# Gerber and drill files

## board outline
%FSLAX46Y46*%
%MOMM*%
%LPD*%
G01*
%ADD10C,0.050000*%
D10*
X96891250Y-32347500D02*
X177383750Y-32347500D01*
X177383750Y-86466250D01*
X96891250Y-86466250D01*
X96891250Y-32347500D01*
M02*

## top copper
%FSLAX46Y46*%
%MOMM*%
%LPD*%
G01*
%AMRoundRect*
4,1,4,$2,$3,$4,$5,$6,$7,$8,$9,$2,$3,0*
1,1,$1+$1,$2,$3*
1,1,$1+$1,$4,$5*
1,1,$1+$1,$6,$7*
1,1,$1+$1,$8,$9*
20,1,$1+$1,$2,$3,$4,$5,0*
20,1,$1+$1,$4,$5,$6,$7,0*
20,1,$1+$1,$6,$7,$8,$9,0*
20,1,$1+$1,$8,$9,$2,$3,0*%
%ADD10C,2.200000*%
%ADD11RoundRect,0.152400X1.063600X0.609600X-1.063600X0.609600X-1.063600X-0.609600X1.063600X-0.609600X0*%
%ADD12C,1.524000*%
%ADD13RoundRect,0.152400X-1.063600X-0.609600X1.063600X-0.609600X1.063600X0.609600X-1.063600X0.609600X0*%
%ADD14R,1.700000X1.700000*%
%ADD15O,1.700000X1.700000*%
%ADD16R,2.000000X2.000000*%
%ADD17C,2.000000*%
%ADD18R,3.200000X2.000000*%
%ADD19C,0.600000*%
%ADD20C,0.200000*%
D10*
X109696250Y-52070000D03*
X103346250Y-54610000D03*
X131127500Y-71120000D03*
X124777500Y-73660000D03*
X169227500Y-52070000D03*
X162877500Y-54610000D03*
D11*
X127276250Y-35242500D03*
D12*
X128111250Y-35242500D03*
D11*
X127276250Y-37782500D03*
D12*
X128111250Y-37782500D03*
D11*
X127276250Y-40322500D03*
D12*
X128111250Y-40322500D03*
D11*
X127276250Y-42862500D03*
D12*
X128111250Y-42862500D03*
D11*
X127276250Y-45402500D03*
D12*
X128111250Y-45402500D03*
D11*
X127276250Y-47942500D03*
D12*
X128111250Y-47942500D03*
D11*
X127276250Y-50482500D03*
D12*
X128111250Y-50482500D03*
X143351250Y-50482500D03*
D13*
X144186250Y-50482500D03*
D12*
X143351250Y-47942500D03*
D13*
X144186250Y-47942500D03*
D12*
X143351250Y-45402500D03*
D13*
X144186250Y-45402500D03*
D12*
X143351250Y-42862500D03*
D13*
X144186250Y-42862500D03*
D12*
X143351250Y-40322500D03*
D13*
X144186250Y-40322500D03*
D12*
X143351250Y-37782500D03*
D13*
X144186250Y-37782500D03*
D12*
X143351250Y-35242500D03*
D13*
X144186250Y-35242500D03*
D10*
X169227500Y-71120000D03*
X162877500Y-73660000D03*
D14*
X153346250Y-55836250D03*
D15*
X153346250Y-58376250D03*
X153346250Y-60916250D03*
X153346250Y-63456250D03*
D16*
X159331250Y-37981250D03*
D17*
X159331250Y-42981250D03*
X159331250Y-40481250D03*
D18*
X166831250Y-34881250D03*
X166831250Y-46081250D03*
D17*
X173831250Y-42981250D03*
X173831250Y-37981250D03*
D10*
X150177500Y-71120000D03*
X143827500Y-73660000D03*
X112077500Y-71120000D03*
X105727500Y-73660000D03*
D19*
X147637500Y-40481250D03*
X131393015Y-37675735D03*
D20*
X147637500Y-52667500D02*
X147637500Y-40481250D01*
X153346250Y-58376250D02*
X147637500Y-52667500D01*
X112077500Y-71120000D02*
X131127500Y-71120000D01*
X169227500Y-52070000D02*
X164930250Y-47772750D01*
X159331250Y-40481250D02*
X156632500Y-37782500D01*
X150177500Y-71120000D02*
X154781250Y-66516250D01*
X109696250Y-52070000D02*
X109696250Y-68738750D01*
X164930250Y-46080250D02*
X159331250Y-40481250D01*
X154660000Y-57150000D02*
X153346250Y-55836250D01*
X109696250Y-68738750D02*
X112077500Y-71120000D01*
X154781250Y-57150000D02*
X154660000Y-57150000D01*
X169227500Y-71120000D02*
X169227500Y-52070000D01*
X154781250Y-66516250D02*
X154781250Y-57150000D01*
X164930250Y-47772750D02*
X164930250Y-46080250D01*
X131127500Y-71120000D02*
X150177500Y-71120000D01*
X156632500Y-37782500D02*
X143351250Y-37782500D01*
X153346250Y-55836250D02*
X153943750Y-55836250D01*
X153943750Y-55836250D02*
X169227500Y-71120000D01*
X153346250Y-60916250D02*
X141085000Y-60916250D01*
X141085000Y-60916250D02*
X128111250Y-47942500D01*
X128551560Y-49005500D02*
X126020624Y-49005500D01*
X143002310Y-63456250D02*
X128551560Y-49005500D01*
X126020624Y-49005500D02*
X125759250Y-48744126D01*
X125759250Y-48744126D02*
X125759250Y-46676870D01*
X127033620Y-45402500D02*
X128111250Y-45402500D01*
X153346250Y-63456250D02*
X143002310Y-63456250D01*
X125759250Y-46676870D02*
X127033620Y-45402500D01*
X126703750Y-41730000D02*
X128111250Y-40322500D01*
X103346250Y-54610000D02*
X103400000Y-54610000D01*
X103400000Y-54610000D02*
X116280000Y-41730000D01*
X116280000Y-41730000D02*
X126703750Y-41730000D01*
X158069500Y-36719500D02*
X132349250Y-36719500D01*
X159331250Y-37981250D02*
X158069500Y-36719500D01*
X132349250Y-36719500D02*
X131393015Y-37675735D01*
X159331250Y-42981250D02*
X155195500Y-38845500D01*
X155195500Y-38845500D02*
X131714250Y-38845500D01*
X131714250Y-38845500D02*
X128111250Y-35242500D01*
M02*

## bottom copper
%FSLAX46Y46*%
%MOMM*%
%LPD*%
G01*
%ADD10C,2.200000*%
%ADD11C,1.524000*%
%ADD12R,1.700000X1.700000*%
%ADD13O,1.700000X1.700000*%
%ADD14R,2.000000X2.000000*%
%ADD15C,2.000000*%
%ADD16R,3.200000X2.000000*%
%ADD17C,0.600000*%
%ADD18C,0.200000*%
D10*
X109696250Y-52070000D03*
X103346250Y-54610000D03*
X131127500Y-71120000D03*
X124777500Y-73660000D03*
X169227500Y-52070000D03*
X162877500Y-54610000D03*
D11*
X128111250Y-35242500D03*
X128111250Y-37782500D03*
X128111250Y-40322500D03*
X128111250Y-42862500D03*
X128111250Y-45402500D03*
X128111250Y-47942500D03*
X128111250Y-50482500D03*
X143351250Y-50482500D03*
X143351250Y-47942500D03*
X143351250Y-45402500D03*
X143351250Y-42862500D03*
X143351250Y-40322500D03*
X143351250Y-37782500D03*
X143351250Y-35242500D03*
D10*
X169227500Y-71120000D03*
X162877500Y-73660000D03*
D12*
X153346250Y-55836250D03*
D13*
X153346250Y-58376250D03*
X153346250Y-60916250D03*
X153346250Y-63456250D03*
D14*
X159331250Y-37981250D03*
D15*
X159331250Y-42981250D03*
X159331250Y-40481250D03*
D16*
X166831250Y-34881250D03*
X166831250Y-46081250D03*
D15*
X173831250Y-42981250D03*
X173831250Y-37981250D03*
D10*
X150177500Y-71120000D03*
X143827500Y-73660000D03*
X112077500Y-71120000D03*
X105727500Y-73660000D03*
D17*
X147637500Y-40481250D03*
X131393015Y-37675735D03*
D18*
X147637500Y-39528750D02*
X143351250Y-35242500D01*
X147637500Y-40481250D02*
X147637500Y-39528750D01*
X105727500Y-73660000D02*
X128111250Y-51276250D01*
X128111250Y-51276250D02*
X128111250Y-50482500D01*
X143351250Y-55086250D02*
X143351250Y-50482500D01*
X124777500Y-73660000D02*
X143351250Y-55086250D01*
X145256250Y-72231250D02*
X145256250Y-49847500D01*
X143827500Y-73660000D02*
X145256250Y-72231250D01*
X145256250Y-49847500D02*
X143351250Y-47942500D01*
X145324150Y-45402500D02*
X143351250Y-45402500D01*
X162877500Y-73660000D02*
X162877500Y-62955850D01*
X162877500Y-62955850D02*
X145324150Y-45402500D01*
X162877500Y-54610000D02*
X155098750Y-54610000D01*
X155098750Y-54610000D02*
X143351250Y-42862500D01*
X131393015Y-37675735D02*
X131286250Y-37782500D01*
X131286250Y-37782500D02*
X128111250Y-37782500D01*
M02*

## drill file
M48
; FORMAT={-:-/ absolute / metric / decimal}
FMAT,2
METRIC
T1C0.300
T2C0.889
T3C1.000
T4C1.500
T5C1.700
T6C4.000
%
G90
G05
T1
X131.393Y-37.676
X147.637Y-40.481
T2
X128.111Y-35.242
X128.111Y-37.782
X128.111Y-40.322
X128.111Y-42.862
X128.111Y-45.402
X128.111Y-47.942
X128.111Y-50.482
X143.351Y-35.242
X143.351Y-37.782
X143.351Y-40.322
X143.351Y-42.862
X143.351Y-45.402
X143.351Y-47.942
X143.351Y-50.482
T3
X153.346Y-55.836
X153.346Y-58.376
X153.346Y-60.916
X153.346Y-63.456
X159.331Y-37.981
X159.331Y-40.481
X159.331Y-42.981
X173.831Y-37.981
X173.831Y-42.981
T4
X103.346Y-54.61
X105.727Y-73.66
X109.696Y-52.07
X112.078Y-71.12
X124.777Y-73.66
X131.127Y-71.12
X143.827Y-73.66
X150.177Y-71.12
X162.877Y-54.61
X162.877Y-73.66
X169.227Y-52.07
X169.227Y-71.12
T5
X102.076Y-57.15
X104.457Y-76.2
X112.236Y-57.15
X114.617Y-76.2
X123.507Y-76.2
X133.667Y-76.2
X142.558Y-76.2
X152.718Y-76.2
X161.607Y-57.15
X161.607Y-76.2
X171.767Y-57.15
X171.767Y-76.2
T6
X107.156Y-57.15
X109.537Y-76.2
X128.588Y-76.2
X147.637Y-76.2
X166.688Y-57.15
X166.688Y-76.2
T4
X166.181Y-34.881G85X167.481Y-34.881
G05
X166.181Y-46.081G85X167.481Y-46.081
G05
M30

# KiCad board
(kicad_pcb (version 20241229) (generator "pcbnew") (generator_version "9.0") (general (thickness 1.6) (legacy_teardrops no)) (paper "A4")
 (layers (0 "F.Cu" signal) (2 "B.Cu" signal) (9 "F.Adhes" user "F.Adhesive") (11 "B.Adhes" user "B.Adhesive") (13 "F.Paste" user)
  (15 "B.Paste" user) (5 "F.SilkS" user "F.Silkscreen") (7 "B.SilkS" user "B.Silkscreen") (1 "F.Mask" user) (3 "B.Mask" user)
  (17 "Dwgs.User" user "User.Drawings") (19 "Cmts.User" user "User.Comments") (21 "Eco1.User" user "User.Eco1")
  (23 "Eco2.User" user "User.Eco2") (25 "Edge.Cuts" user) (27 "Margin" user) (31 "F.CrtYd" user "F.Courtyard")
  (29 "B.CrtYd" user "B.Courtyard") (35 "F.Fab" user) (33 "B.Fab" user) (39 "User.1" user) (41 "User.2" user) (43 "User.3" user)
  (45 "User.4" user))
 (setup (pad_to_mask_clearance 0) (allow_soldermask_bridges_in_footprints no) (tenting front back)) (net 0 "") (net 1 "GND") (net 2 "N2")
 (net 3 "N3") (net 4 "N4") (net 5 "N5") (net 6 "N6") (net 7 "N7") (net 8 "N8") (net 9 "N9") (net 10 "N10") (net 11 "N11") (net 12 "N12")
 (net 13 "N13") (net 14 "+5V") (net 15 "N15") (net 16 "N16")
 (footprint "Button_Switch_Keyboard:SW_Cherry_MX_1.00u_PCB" (layer "F.Cu") (at 109.69625 52.07)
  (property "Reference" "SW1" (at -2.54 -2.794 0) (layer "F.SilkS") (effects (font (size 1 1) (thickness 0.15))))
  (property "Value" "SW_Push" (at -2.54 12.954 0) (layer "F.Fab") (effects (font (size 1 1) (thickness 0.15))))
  (pad "" np_thru_hole circle (at -7.62 5.08) (size 1.7 1.7) (drill 1.7) (layers "*.Cu" "*.Mask"))
  (pad "" np_thru_hole circle (at -2.54 5.08) (size 4 4) (drill 4) (layers "*.Cu" "*.Mask"))
  (pad "" np_thru_hole circle (at 2.54 5.08) (size 1.7 1.7) (drill 1.7) (layers "*.Cu" "*.Mask"))
  (pad "1" thru_hole circle (at 0 0) (size 2.2 2.2) (drill 1.5) (layers "*.Cu" "*.Mask") (remove_unused_layers no) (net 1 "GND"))
  (pad "2" thru_hole circle (at -6.35 2.54) (size 2.2 2.2) (drill 1.5) (layers "*.Cu" "*.Mask") (remove_unused_layers no) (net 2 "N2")))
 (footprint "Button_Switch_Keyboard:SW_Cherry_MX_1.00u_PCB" (layer "F.Cu") (at 131.1275 71.12)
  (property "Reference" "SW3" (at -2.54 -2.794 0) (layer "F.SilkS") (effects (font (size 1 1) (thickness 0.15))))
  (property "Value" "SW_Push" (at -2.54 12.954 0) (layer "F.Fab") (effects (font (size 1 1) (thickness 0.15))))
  (pad "" np_thru_hole circle (at -7.62 5.08) (size 1.7 1.7) (drill 1.7) (layers "*.Cu" "*.Mask"))
  (pad "" np_thru_hole circle (at -2.54 5.08) (size 4 4) (drill 4) (layers "*.Cu" "*.Mask"))
  (pad "" np_thru_hole circle (at 2.54 5.08) (size 1.7 1.7) (drill 1.7) (layers "*.Cu" "*.Mask"))
  (pad "1" thru_hole circle (at 0 0) (size 2.2 2.2) (drill 1.5) (layers "*.Cu" "*.Mask") (remove_unused_layers no) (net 1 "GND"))
  (pad "2" thru_hole circle (at -6.35 2.54) (size 2.2 2.2) (drill 1.5) (layers "*.Cu" "*.Mask") (remove_unused_layers no) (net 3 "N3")))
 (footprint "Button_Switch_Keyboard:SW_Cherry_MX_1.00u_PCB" (layer "F.Cu") (at 169.2275 52.07)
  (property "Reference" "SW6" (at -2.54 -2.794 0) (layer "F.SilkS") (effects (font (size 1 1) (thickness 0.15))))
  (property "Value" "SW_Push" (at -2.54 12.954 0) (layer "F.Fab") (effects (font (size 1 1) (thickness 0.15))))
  (pad "" np_thru_hole circle (at -7.62 5.08) (size 1.7 1.7) (drill 1.7) (layers "*.Cu" "*.Mask"))
  (pad "" np_thru_hole circle (at -2.54 5.08) (size 4 4) (drill 4) (layers "*.Cu" "*.Mask"))
  (pad "" np_thru_hole circle (at 2.54 5.08) (size 1.7 1.7) (drill 1.7) (layers "*.Cu" "*.Mask"))
  (pad "1" thru_hole circle (at 0 0) (size 2.2 2.2) (drill 1.5) (layers "*.Cu" "*.Mask") (remove_unused_layers no) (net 1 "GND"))
  (pad "2" thru_hole circle (at -6.35 2.54) (size 2.2 2.2) (drill 1.5) (layers "*.Cu" "*.Mask") (remove_unused_layers no) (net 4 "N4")))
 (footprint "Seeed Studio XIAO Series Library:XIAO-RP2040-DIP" (layer "F.Cu") (at 135.73125 42.8625)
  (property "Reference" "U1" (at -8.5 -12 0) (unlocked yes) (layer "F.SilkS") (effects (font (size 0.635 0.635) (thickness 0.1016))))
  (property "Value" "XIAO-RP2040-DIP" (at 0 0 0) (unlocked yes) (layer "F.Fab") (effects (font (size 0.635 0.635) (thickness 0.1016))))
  (pad "1" smd roundrect (at -8.455 -7.62 180) (size 2.432 1.524) (layers "F.Cu" "F.Mask") (roundrect_rratio 0.1) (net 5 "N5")
   (thermal_bridge_angle 45))
  (pad "1" thru_hole circle (at -7.62 -7.62 180) (size 1.524 1.524) (drill 0.889) (layers "*.Cu" "*.Mask") (remove_unused_layers no)
   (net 5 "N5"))
  (pad "2" smd roundrect (at -8.455 -5.08 180) (size 2.432 1.524) (layers "F.Cu" "F.Mask") (roundrect_rratio 0.1) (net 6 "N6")
   (thermal_bridge_angle 45))
  (pad "2" thru_hole circle (at -7.62 -5.08 180) (size 1.524 1.524) (drill 0.889) (layers "*.Cu" "*.Mask") (remove_unused_layers no)
   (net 6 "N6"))
  (pad "3" smd roundrect (at -8.455 -2.54 180) (size 2.432 1.524) (layers "F.Cu" "F.Mask") (roundrect_rratio 0.1) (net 2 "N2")
   (thermal_bridge_angle 45))
  (pad "3" thru_hole circle (at -7.62 -2.54 180) (size 1.524 1.524) (drill 0.889) (layers "*.Cu" "*.Mask") (remove_unused_layers no)
   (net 2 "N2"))
  (pad "4" smd roundrect (at -8.455 0 180) (size 2.432 1.524) (layers "F.Cu" "F.Mask") (roundrect_rratio 0.1) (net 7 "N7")
   (thermal_bridge_angle 45))
  (pad "4" thru_hole circle (at -7.62 0 180) (size 1.524 1.524) (drill 0.889) (layers "*.Cu" "*.Mask") (remove_unused_layers no)
   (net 7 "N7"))
  (pad "5" smd roundrect (at -8.455 2.54 180) (size 2.432 1.524) (layers "F.Cu" "F.Mask") (roundrect_rratio 0.1) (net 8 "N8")
   (thermal_bridge_angle 45))
  (pad "5" thru_hole circle (at -7.62 2.54 180) (size 1.524 1.524) (drill 0.889) (layers "*.Cu" "*.Mask") (remove_unused_layers no)
   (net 8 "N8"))
  (pad "6" smd roundrect (at -8.455 5.08 180) (size 2.432 1.524) (layers "F.Cu" "F.Mask") (roundrect_rratio 0.1) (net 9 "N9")
   (thermal_bridge_angle 45))
  (pad "6" thru_hole circle (at -7.62 5.08 180) (size 1.524 1.524) (drill 0.889) (layers "*.Cu" "*.Mask") (remove_unused_layers no)
   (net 9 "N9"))
  (pad "7" smd roundrect (at -8.455 7.62 180) (size 2.432 1.524) (layers "F.Cu" "F.Mask") (roundrect_rratio 0.1) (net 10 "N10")
   (thermal_bridge_angle 45))
  (pad "7" thru_hole circle (at -7.62 7.62 180) (size 1.524 1.524) (drill 0.889) (layers "*.Cu" "*.Mask") (remove_unused_layers no)
   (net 10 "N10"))
  (pad "8" thru_hole circle (at 7.62 7.62) (size 1.524 1.524) (drill 0.889) (layers "*.Cu" "*.Mask") (remove_unused_layers no) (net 3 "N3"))
  (pad "8" smd roundrect (at 8.455 7.62) (size 2.432 1.524) (layers "F.Cu" "F.Mask") (roundrect_rratio 0.1) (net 3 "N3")
   (thermal_bridge_angle 45))
  (pad "9" thru_hole circle (at 7.62 5.08) (size 1.524 1.524) (drill 0.889) (layers "*.Cu" "*.Mask") (remove_unused_layers no)
   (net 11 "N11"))
  (pad "9" smd roundrect (at 8.455 5.08) (size 2.432 1.524) (layers "F.Cu" "F.Mask") (roundrect_rratio 0.1) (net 11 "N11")
   (thermal_bridge_angle 45))
  (pad "10" thru_hole circle (at 7.62 2.54) (size 1.524 1.524) (drill 0.889) (layers "*.Cu" "*.Mask") (remove_unused_layers no)
   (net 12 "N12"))
  (pad "10" smd roundrect (at 8.455 2.54) (size 2.432 1.524) (layers "F.Cu" "F.Mask") (roundrect_rratio 0.1) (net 12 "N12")
   (thermal_bridge_angle 45))
  (pad "11" thru_hole circle (at 7.62 0) (size 1.524 1.524) (drill 0.889) (layers "*.Cu" "*.Mask") (remove_unused_layers no) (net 4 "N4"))
  (pad "11" smd roundrect (at 8.455 0) (size 2.432 1.524) (layers "F.Cu" "F.Mask") (roundrect_rratio 0.1) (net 4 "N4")
   (thermal_bridge_angle 45))
  (pad "12" thru_hole circle (at 7.62 -2.54) (size 1.524 1.524) (drill 0.889) (layers "*.Cu" "*.Mask") (remove_unused_layers no)
   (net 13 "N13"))
  (pad "12" smd roundrect (at 8.455 -2.54) (size 2.432 1.524) (layers "F.Cu" "F.Mask") (roundrect_rratio 0.1) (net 13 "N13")
   (thermal_bridge_angle 45))
  (pad "13" thru_hole circle (at 7.62 -5.08) (size 1.524 1.524) (drill 0.889) (layers "*.Cu" "*.Mask") (remove_unused_layers no)
   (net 1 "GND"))
  (pad "13" smd roundrect (at 8.455 -5.08) (size 2.432 1.524) (layers "F.Cu" "F.Mask") (roundrect_rratio 0.1) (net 1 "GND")
   (thermal_bridge_angle 45))
  (pad "14" thru_hole circle (at 7.62 -7.62) (size 1.524 1.524) (drill 0.889) (layers "*.Cu" "*.Mask") (remove_unused_layers no)
   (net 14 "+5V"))
  (pad "14" smd roundrect (at 8.455 -7.62) (size 2.432 1.524) (layers "F.Cu" "F.Mask") (roundrect_rratio 0.1) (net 14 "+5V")
   (thermal_bridge_angle 45)))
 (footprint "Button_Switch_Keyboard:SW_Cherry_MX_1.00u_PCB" (layer "F.Cu") (at 169.2275 71.12)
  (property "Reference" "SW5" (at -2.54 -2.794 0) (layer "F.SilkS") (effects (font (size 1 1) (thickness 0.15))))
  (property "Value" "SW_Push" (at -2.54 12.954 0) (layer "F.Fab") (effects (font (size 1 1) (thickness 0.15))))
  (pad "" np_thru_hole circle (at -7.62 5.08) (size 1.7 1.7) (drill 1.7) (layers "*.Cu" "*.Mask"))
  (pad "" np_thru_hole circle (at -2.54 5.08) (size 4 4) (drill 4) (layers "*.Cu" "*.Mask"))
  (pad "" np_thru_hole circle (at 2.54 5.08) (size 1.7 1.7) (drill 1.7) (layers "*.Cu" "*.Mask"))
  (pad "1" thru_hole circle (at 0 0) (size 2.2 2.2) (drill 1.5) (layers "*.Cu" "*.Mask") (remove_unused_layers no) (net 1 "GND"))
  (pad "2" thru_hole circle (at -6.35 2.54) (size 2.2 2.2) (drill 1.5) (layers "*.Cu" "*.Mask") (remove_unused_layers no) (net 12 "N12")))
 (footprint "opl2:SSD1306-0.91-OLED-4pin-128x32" (layer "F.Cu") (at 116.84625 53.64625)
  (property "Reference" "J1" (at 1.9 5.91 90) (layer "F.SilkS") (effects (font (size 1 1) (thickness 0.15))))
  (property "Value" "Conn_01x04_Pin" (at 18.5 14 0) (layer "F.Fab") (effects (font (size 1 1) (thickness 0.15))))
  (pad "1" thru_hole rect (at 36.5 2.19) (size 1.7 1.7) (drill 1) (layers "*.Cu" "*.Mask") (remove_unused_layers no) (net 1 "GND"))
  (pad "2" thru_hole oval (at 36.5 4.73) (size 1.7 1.7) (drill 1) (layers "*.Cu" "*.Mask") (remove_unused_layers no) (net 14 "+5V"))
  (pad "3" thru_hole oval (at 36.5 7.27) (size 1.7 1.7) (drill 1) (layers "*.Cu" "*.Mask") (remove_unused_layers no) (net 9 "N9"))
  (pad "4" thru_hole oval (at 36.5 9.81) (size 1.7 1.7) (drill 1) (layers "*.Cu" "*.Mask") (remove_unused_layers no) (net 8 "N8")))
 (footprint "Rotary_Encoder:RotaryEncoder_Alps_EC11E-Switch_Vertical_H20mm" (layer "F.Cu") (at 159.33125 37.98125)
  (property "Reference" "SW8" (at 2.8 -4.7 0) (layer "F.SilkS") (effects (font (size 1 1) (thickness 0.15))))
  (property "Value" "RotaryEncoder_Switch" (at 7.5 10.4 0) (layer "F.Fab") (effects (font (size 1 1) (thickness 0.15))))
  (pad "A" thru_hole rect (at 0 0) (size 2 2) (drill 1) (layers "*.Cu" "*.Mask") (remove_unused_layers no) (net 6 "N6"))
  (pad "B" thru_hole circle (at 0 5) (size 2 2) (drill 1) (layers "*.Cu" "*.Mask") (remove_unused_layers no) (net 5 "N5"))
  (pad "C" thru_hole circle (at 0 2.5) (size 2 2) (drill 1) (layers "*.Cu" "*.Mask") (remove_unused_layers no) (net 1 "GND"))
  (pad "MP" thru_hole rect (at 7.5 -3.1) (size 3.2 2) (drill oval 2.8 1.5) (layers "*.Cu" "*.Mask") (remove_unused_layers no))
  (pad "MP" thru_hole rect (at 7.5 8.1) (size 3.2 2) (drill oval 2.8 1.5) (layers "*.Cu" "*.Mask") (remove_unused_layers no))
  (pad "S1" thru_hole circle (at 14.5 5) (size 2 2) (drill 1) (layers "*.Cu" "*.Mask") (remove_unused_layers no) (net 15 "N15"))
  (pad "S2" thru_hole circle (at 14.5 0) (size 2 2) (drill 1) (layers "*.Cu" "*.Mask") (remove_unused_layers no) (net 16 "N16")))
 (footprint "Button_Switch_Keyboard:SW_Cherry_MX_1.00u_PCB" (layer "F.Cu") (at 150.1775 71.12)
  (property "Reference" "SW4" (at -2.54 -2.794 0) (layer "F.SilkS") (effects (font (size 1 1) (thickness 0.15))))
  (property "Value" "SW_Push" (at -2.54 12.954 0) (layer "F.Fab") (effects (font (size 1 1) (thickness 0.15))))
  (pad "" np_thru_hole circle (at -7.62 5.08) (size 1.7 1.7) (drill 1.7) (layers "*.Cu" "*.Mask"))
  (pad "" np_thru_hole circle (at -2.54 5.08) (size 4 4) (drill 4) (layers "*.Cu" "*.Mask"))
  (pad "" np_thru_hole circle (at 2.54 5.08) (size 1.7 1.7) (drill 1.7) (layers "*.Cu" "*.Mask"))
  (pad "1" thru_hole circle (at 0 0) (size 2.2 2.2) (drill 1.5) (layers "*.Cu" "*.Mask") (remove_unused_layers no) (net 1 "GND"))
  (pad "2" thru_hole circle (at -6.35 2.54) (size 2.2 2.2) (drill 1.5) (layers "*.Cu" "*.Mask") (remove_unused_layers no) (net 11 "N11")))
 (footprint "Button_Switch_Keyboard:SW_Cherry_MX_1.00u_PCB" (layer "F.Cu") (at 112.0775 71.12)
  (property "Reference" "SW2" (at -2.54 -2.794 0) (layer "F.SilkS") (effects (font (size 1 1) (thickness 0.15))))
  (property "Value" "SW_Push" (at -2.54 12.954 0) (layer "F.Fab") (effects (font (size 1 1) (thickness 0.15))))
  (pad "" np_thru_hole circle (at -7.62 5.08) (size 1.7 1.7) (drill 1.7) (layers "*.Cu" "*.Mask"))
  (pad "" np_thru_hole circle (at -2.54 5.08) (size 4 4) (drill 4) (layers "*.Cu" "*.Mask"))
  (pad "" np_thru_hole circle (at 2.54 5.08) (size 1.7 1.7) (drill 1.7) (layers "*.Cu" "*.Mask"))
  (pad "1" thru_hole circle (at 0 0) (size 2.2 2.2) (drill 1.5) (layers "*.Cu" "*.Mask") (remove_unused_layers no) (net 1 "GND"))
  (pad "2" thru_hole circle (at -6.35 2.54) (size 2.2 2.2) (drill 1.5) (layers "*.Cu" "*.Mask") (remove_unused_layers no) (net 10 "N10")))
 (gr_rect (start 96.89125 32.3475) (end 177.38375 86.46625) (stroke (width 0.05) (type default)) (fill no) (layer "Edge.Cuts"))
 (segment (start 147.6375 52.6675) (end 147.6375 40.48125) (width 0.2) (layer "F.Cu") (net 14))
 (segment (start 153.34625 58.37625) (end 147.6375 52.6675) (width 0.2) (layer "F.Cu") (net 14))
 (via (at 147.6375 40.48125) (size 0.6) (drill 0.3) (layers "F.Cu" "B.Cu") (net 14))
 (segment (start 147.6375 39.52875) (end 143.35125 35.2425) (width 0.2) (layer "B.Cu") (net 14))
 (segment (start 147.6375 40.48125) (end 147.6375 39.52875) (width 0.2) (layer "B.Cu") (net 14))
 (segment (start 112.0775 71.12) (end 131.1275 71.12) (width 0.2) (layer "F.Cu") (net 1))
 (segment (start 169.2275 52.07) (end 164.93025 47.77275) (width 0.2) (layer "F.Cu") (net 1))
 (segment (start 159.33125 40.48125) (end 156.6325 37.7825) (width 0.2) (layer "F.Cu") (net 1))
 (segment (start 150.1775 71.12) (end 154.78125 66.51625) (width 0.2) (layer "F.Cu") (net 1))
 (segment (start 109.69625 52.07) (end 109.69625 68.73875) (width 0.2) (layer "F.Cu") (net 1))
 (segment (start 164.93025 46.08025) (end 159.33125 40.48125) (width 0.2) (layer "F.Cu") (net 1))
 (segment (start 154.66 57.15) (end 153.34625 55.83625) (width 0.2) (layer "F.Cu") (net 1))
 (segment (start 109.69625 68.73875) (end 112.0775 71.12) (width 0.2) (layer "F.Cu") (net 1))
 (segment (start 154.78125 57.15) (end 154.66 57.15) (width 0.2) (layer "F.Cu") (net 1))
 (segment (start 169.2275 71.12) (end 169.2275 52.07) (width 0.2) (layer "F.Cu") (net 1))
 (segment (start 154.78125 66.51625) (end 154.78125 57.15) (width 0.2) (layer "F.Cu") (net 1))
 (segment (start 164.93025 47.77275) (end 164.93025 46.08025) (width 0.2) (layer "F.Cu") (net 1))
 (segment (start 131.1275 71.12) (end 150.1775 71.12) (width 0.2) (layer "F.Cu") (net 1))
 (segment (start 156.6325 37.7825) (end 143.35125 37.7825) (width 0.2) (layer "F.Cu") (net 1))
 (segment (start 153.34625 55.83625) (end 153.94375 55.83625) (width 0.2) (layer "F.Cu") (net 1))
 (segment (start 153.94375 55.83625) (end 169.2275 71.12) (width 0.2) (layer "F.Cu") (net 1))
 (segment (start 153.34625 60.91625) (end 141.085 60.91625) (width 0.2) (layer "F.Cu") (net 9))
 (segment (start 141.085 60.91625) (end 128.11125 47.9425) (width 0.2) (layer "F.Cu") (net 9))
 (segment (start 128.55156 49.0055) (end 126.020624 49.0055) (width 0.2) (layer "F.Cu") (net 8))
 (segment (start 143.00231 63.45625) (end 128.55156 49.0055) (width 0.2) (layer "F.Cu") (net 8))
 (segment (start 126.020624 49.0055) (end 125.75925 48.744126) (width 0.2) (layer "F.Cu") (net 8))
 (segment (start 125.75925 48.744126) (end 125.75925 46.67687) (width 0.2) (layer "F.Cu") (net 8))
 (segment (start 127.03362 45.4025) (end 128.11125 45.4025) (width 0.2) (layer "F.Cu") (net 8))
 (segment (start 153.34625 63.45625) (end 143.00231 63.45625) (width 0.2) (layer "F.Cu") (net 8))
 (segment (start 125.75925 46.67687) (end 127.03362 45.4025) (width 0.2) (layer "F.Cu") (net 8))
 (segment (start 126.70375 41.73) (end 128.11125 40.3225) (width 0.2) (layer "F.Cu") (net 2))
 (segment (start 103.34625 54.61) (end 103.4 54.61) (width 0.2) (layer "F.Cu") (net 2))
 (segment (start 103.4 54.61) (end 116.28 41.73) (width 0.2) (layer "F.Cu") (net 2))
 (segment (start 116.28 41.73) (end 126.70375 41.73) (width 0.2) (layer "F.Cu") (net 2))
 (segment (start 105.7275 73.66) (end 128.11125 51.27625) (width 0.2) (layer "B.Cu") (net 10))
 (segment (start 128.11125 51.27625) (end 128.11125 50.4825) (width 0.2) (layer "B.Cu") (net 10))
 (segment (start 143.35125 55.08625) (end 143.35125 50.4825) (width 0.2) (layer "B.Cu") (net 3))
 (segment (start 124.7775 73.66) (end 143.35125 55.08625) (width 0.2) (layer "B.Cu") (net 3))
 (segment (start 145.25625 72.23125) (end 145.25625 49.8475) (width 0.2) (layer "B.Cu") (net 11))
 (segment (start 143.8275 73.66) (end 145.25625 72.23125) (width 0.2) (layer "B.Cu") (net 11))
 (segment (start 145.25625 49.8475) (end 143.35125 47.9425) (width 0.2) (layer "B.Cu") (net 11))
 (segment (start 145.32415 45.4025) (end 143.35125 45.4025) (width 0.2) (layer "B.Cu") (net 12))
 (segment (start 162.8775 73.66) (end 162.8775 62.95585) (width 0.2) (layer "B.Cu") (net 12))
 (segment (start 162.8775 62.95585) (end 145.32415 45.4025) (width 0.2) (layer "B.Cu") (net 12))
 (segment (start 162.8775 54.61) (end 155.09875 54.61) (width 0.2) (layer "B.Cu") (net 4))
 (segment (start 155.09875 54.61) (end 143.35125 42.8625) (width 0.2) (layer "B.Cu") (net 4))
 (segment (start 158.0695 36.7195) (end 132.34925 36.7195) (width 0.2) (layer "F.Cu") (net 6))
 (segment (start 159.33125 37.98125) (end 158.0695 36.7195) (width 0.2) (layer "F.Cu") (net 6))
 (segment (start 132.34925 36.7195) (end 131.393015 37.675735) (width 0.2) (layer "F.Cu") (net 6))
 (via (at 131.393015 37.675735) (size 0.6) (drill 0.3) (layers "F.Cu" "B.Cu") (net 6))
 (segment (start 131.393015 37.675735) (end 131.28625 37.7825) (width 0.2) (layer "B.Cu") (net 6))
 (segment (start 131.28625 37.7825) (end 128.11125 37.7825) (width 0.2) (layer "B.Cu") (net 6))
 (segment (start 159.33125 42.98125) (end 155.1955 38.8455) (width 0.2) (layer "F.Cu") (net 5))
 (segment (start 155.1955 38.8455) (end 131.71425 38.8455) (width 0.2) (layer "F.Cu") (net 5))
 (segment (start 131.71425 38.8455) (end 128.11125 35.2425) (width 0.2) (layer "F.Cu") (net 5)))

